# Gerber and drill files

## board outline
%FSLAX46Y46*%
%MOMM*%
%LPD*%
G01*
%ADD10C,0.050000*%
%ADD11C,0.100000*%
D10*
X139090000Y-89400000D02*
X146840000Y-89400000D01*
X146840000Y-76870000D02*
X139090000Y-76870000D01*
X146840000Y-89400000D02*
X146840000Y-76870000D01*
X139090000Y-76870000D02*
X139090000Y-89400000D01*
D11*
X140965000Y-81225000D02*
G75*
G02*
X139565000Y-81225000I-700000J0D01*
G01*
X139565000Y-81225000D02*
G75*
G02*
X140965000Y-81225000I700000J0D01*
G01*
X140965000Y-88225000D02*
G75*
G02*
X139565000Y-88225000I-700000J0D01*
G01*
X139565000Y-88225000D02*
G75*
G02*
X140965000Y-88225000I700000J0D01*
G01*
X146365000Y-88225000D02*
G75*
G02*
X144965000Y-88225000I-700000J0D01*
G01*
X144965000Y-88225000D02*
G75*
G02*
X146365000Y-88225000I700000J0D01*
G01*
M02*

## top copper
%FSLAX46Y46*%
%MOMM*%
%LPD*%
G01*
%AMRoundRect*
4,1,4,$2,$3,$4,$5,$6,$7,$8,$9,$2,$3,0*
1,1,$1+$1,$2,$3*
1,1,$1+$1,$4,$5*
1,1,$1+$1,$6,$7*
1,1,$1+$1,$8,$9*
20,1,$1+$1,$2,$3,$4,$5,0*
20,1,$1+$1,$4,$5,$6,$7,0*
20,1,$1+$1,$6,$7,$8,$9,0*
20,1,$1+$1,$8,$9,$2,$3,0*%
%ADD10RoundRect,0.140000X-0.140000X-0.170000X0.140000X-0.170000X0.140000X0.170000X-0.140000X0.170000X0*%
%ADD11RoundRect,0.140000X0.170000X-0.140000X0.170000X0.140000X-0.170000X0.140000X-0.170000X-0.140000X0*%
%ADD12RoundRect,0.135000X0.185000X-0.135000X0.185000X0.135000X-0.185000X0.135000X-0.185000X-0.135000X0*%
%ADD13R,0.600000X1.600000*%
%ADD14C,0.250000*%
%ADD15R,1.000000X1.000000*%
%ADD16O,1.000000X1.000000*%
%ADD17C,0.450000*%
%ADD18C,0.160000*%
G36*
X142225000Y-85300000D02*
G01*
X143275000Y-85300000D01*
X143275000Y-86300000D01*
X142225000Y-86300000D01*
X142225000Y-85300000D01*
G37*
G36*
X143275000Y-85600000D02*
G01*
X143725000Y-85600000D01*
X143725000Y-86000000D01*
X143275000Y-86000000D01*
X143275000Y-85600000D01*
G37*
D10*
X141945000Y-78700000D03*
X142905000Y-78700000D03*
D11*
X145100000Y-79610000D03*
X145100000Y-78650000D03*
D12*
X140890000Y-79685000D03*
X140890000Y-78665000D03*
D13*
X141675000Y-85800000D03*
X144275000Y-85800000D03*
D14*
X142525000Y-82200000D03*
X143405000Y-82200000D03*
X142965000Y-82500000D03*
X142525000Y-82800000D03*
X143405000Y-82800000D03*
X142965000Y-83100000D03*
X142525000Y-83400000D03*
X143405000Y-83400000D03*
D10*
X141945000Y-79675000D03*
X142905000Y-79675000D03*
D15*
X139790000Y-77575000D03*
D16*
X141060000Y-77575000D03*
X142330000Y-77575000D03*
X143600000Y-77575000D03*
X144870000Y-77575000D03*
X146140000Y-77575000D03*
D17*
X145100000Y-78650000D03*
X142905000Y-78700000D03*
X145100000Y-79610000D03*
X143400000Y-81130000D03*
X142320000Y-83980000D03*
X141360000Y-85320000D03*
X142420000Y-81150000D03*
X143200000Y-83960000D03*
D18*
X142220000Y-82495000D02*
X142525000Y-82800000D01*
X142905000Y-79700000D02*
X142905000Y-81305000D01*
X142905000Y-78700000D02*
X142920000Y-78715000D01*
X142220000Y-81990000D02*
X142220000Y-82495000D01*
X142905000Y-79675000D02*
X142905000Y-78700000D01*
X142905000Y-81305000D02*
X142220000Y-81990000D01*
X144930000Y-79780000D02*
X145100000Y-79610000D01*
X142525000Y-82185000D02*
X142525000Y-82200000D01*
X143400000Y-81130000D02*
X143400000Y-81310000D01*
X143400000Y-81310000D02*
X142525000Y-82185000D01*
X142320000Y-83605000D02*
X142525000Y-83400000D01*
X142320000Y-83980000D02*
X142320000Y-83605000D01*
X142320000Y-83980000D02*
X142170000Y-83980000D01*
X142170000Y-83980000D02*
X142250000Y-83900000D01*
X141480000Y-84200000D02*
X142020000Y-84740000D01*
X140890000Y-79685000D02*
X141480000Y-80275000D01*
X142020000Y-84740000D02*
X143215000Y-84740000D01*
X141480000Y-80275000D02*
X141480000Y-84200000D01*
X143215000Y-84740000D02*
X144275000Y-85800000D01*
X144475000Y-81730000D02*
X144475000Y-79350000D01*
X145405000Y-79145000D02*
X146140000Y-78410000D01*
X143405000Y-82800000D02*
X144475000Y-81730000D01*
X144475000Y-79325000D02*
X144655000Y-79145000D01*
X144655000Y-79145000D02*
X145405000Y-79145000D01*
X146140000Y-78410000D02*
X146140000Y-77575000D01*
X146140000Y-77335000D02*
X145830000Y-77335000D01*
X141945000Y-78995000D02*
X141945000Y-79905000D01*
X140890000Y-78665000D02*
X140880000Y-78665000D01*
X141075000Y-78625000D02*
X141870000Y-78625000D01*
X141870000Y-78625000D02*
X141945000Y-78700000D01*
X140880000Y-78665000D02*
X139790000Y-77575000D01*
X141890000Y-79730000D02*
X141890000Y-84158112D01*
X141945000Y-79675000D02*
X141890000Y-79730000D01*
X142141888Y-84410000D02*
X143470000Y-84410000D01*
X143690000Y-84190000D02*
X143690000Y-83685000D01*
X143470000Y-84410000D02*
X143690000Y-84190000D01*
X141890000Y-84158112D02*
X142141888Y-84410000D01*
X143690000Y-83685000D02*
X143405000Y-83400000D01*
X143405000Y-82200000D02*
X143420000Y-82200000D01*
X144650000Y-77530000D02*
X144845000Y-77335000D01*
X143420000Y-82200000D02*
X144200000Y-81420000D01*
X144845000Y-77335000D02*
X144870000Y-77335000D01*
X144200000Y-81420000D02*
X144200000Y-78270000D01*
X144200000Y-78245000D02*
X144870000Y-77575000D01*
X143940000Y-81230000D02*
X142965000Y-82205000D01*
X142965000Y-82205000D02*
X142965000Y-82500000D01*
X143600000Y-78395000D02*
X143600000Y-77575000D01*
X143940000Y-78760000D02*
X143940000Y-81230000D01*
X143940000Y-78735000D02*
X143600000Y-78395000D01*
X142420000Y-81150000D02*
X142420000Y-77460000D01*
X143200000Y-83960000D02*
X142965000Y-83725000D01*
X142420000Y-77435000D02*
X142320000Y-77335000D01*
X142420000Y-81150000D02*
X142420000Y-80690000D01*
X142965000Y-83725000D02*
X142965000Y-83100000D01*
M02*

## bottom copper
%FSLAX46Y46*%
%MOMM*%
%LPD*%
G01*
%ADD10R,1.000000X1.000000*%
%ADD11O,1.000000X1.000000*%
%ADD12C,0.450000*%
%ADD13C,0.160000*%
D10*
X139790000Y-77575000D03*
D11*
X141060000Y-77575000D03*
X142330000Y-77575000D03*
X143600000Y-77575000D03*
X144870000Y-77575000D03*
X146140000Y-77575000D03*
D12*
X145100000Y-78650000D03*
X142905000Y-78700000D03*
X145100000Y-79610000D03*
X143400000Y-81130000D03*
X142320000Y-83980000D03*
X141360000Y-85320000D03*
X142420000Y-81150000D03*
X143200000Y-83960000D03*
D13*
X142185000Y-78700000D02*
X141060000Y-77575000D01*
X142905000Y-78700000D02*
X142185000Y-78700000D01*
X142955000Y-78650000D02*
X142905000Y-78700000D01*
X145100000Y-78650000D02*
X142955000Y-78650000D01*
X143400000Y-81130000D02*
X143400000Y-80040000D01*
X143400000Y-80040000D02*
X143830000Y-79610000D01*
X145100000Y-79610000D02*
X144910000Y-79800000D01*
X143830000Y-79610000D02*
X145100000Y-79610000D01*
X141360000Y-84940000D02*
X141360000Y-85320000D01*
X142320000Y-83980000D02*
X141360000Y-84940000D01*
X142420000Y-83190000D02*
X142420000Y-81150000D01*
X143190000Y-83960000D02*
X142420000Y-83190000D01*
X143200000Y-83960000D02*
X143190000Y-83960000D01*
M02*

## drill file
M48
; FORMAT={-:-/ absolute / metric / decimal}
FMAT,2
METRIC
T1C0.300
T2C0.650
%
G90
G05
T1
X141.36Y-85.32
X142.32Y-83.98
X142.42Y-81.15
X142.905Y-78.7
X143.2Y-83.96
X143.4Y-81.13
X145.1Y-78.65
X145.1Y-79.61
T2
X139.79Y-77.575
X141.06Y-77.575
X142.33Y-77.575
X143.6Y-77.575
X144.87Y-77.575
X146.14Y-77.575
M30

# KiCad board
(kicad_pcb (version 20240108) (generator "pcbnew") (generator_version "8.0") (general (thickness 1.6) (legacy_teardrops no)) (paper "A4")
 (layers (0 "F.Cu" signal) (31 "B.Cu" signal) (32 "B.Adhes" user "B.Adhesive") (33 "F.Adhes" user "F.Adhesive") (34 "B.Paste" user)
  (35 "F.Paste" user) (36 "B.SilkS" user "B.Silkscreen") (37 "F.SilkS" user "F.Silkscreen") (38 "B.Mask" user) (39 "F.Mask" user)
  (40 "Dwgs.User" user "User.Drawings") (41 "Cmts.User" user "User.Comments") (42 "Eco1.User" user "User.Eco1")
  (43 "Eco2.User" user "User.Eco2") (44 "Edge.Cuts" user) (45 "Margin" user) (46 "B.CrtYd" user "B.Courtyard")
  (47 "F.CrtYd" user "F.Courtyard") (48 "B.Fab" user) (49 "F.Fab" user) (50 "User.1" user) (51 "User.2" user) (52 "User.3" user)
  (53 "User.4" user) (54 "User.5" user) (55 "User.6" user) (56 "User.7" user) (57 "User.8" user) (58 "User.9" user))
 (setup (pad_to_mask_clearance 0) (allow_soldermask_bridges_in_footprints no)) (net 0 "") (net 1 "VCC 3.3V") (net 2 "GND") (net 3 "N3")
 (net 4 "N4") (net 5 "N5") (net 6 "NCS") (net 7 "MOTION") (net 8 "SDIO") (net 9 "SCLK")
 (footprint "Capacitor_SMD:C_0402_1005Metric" (layer "F.Cu") (at 142.425 78.7)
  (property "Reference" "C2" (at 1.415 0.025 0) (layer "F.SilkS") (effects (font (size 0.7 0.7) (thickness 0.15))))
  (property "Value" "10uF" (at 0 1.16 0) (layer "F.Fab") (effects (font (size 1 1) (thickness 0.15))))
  (pad "1" smd roundrect (at -0.48 0) (size 0.56 0.62) (layers "F.Cu" "F.Paste" "F.Mask") (roundrect_rratio 0.25) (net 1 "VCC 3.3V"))
  (pad "2" smd roundrect (at 0.48 0) (size 0.56 0.62) (layers "F.Cu" "F.Paste" "F.Mask") (roundrect_rratio 0.25) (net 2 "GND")))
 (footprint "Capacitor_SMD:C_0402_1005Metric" (layer "F.Cu") (at 145.1 79.13 90)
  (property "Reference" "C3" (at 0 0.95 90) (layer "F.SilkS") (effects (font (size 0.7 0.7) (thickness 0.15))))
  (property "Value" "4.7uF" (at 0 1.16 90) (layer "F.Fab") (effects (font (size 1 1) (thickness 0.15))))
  (pad "1" smd roundrect (at -0.48 0 90) (size 0.56 0.62) (layers "F.Cu" "F.Paste" "F.Mask") (roundrect_rratio 0.25) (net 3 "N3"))
  (pad "2" smd roundrect (at 0.48 0 90) (size 0.56 0.62) (layers "F.Cu" "F.Paste" "F.Mask") (roundrect_rratio 0.25) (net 2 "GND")))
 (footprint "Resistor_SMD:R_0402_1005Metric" (layer "F.Cu") (at 140.89 79.175 90)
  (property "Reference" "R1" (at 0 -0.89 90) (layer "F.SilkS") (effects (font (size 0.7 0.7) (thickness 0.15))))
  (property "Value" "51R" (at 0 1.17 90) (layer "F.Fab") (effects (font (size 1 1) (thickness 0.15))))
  (pad "1" smd roundrect (at -0.51 0 90) (size 0.54 0.64) (layers "F.Cu" "F.Paste" "F.Mask") (roundrect_rratio 0.25) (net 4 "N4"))
  (pad "2" smd roundrect (at 0.51 0 90) (size 0.54 0.64) (layers "F.Cu" "F.Paste" "F.Mask") (roundrect_rratio 0.25) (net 1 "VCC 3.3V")))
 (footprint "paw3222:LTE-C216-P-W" (layer "F.Cu") (at 142.975 85.8 90)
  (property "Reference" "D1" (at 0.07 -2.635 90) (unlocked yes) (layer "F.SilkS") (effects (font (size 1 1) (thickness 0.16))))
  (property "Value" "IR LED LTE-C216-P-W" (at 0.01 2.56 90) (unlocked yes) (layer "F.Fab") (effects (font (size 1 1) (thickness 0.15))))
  (fp_rect (start -0.5 -0.75) (end 0.5 0.3) (stroke (width 0) (type solid)) (fill solid) (layer "F.Cu"))
  (fp_rect (start -0.2 0.3) (end 0.2 0.75) (stroke (width 0) (type solid)) (fill solid) (layer "F.Cu"))
  (pad "1" smd rect (at 0 -1.3 90) (size 1.6 0.6) (layers "F.Cu" "F.Paste" "F.Mask") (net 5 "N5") (thermal_bridge_angle 45))
  (pad "2" smd rect (at 0 1.3 90) (size 1.6 0.6) (layers "F.Cu" "F.Paste" "F.Mask") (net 4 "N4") (thermal_bridge_angle 45)))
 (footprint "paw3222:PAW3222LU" (layer "F.Cu") (at 142.965 82.8)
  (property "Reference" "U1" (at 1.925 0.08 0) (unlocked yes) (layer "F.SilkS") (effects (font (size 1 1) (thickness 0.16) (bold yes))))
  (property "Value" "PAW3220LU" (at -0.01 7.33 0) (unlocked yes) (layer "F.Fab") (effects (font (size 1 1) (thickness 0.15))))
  (fp_circle (center -2.7 -1.575) (end -2 -1.575) (stroke (width 0.1) (type default)) (fill none) (layer "Edge.Cuts"))
  (fp_circle (center -2.7 5.425) (end -2 5.425) (stroke (width 0.1) (type default)) (fill none) (layer "Edge.Cuts"))
  (fp_circle (center 2.7 5.425) (end 3.4 5.425) (stroke (width 0.1) (type default)) (fill none) (layer "Edge.Cuts"))
  (pad "A1" smd circle (at -0.44 -0.6) (size 0.25 0.25) (layers "F.Cu" "F.Paste" "F.Mask") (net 3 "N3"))
  (pad "A3" smd circle (at 0.44 -0.6) (size 0.25 0.25) (layers "F.Cu" "F.Paste" "F.Mask") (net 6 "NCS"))
  (pad "B2" smd circle (at 0 -0.3) (size 0.25 0.25) (layers "F.Cu" "F.Paste" "F.Mask") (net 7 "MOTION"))
  (pad "C1" smd circle (at -0.44 0) (size 0.25 0.25) (layers "F.Cu" "F.Paste" "F.Mask") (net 2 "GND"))
  (pad "C3" smd circle (at 0.44 0) (size 0.25 0.25) (layers "F.Cu" "F.Paste" "F.Mask") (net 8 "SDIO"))
  (pad "D2" smd circle (at 0 0.3) (size 0.25 0.25) (layers "F.Cu" "F.Paste" "F.Mask") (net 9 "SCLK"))
  (pad "E1" smd circle (at -0.44 0.6) (size 0.25 0.25) (layers "F.Cu" "F.Paste" "F.Mask") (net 5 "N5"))
  (pad "E3" smd circle (at 0.44 0.6) (size 0.25 0.25) (layers "F.Cu" "F.Paste" "F.Mask") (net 1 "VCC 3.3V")))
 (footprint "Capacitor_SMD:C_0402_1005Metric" (layer "F.Cu") (at 142.425 79.675)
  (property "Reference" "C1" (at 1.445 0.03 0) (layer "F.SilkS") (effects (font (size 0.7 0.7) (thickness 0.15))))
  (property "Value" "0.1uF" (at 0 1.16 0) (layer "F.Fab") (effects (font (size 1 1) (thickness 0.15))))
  (pad "1" smd roundrect (at -0.48 0) (size 0.56 0.62) (layers "F.Cu" "F.Paste" "F.Mask") (roundrect_rratio 0.25) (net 1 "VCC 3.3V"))
  (pad "2" smd roundrect (at 0.48 0) (size 0.56 0.62) (layers "F.Cu" "F.Paste" "F.Mask") (roundrect_rratio 0.25) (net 2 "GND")))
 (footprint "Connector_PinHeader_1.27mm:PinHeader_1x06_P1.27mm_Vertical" (layer "F.Cu") (at 139.79 77.575 90)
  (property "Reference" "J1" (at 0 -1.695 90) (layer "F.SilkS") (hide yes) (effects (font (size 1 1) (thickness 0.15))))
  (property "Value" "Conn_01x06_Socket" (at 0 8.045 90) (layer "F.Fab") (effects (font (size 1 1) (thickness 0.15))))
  (pad "1" thru_hole rect (at 0 0 90) (size 1 1) (drill 0.65) (layers "*.Cu" "*.Mask") (remove_unused_layers no) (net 1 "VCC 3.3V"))
  (pad "2" thru_hole oval (at 0 1.27 90) (size 1 1) (drill 0.65) (layers "*.Cu" "*.Mask") (remove_unused_layers no) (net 2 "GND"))
  (pad "3" thru_hole oval (at 0 2.54 90) (size 1 1) (drill 0.65) (layers "*.Cu" "*.Mask") (remove_unused_layers no) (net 9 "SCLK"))
  (pad "4" thru_hole oval (at 0 3.81 90) (size 1 1) (drill 0.65) (layers "*.Cu" "*.Mask") (remove_unused_layers no) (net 7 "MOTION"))
  (pad "5" thru_hole oval (at 0 5.08 90) (size 1 1) (drill 0.65) (layers "*.Cu" "*.Mask") (remove_unused_layers no) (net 6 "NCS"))
  (pad "6" thru_hole oval (at 0 6.35 90) (size 1 1) (drill 0.65) (layers "*.Cu" "*.Mask") (remove_unused_layers no) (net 8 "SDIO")))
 (gr_line (start 139.09 89.4) (end 146.84 89.4) (stroke (width 0.05) (type default)) (layer "Edge.Cuts"))
 (gr_line (start 146.84 76.87) (end 139.09 76.87) (stroke (width 0.05) (type default)) (layer "Edge.Cuts"))
 (gr_line (start 146.84 89.4) (end 146.84 76.87) (stroke (width 0.05) (type default)) (layer "Edge.Cuts"))
 (gr_line (start 139.09 76.87) (end 139.09 89.4) (stroke (width 0.05) (type default)) (layer "Edge.Cuts"))
 (segment (start 142.22 82.495) (end 142.525 82.8) (width 0.16) (layer "F.Cu") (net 2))
 (segment (start 142.905 79.7) (end 142.905 81.305) (width 0.16) (layer "F.Cu") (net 2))
 (segment (start 142.905 78.7) (end 142.92 78.715) (width 0.16) (layer "F.Cu") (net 2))
 (segment (start 142.22 81.99) (end 142.22 82.495) (width 0.16) (layer "F.Cu") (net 2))
 (segment (start 142.905 79.675) (end 142.905 78.7) (width 0.16) (layer "F.Cu") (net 2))
 (segment (start 142.905 81.305) (end 142.22 81.99) (width 0.16) (layer "F.Cu") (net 2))
 (via (at 145.1 78.65) (size 0.45) (drill 0.3) (layers "F.Cu" "B.Cu") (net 2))
 (via (at 142.905 78.7) (size 0.45) (drill 0.3) (layers "F.Cu" "B.Cu") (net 2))
 (segment (start 142.185 78.7) (end 141.06 77.575) (width 0.16) (layer "B.Cu") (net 2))
 (segment (start 142.905 78.7) (end 142.185 78.7) (width 0.16) (layer "B.Cu") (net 2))
 (segment (start 142.955 78.65) (end 142.905 78.7) (width 0.16) (layer "B.Cu") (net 2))
 (segment (start 145.1 78.65) (end 142.955 78.65) (width 0.16) (layer "B.Cu") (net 2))
 (segment (start 144.93 79.78) (end 145.1 79.61) (width 0.16) (layer "F.Cu") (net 3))
 (segment (start 142.525 82.185) (end 142.525 82.2) (width 0.16) (layer "F.Cu") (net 3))
 (segment (start 143.4 81.13) (end 143.4 81.31) (width 0.16) (layer "F.Cu") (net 3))
 (segment (start 143.4 81.31) (end 142.525 82.185) (width 0.16) (layer "F.Cu") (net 3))
 (via (at 145.1 79.61) (size 0.45) (drill 0.3) (layers "F.Cu" "B.Cu") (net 3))
 (via (at 143.4 81.13) (size 0.45) (drill 0.3) (layers "F.Cu" "B.Cu") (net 3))
 (segment (start 143.4 81.13) (end 143.4 80.04) (width 0.16) (layer "B.Cu") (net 3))
 (segment (start 143.4 80.04) (end 143.83 79.61) (width 0.16) (layer "B.Cu") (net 3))
 (segment (start 145.1 79.61) (end 144.91 79.8) (width 0.16) (layer "B.Cu") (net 3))
 (segment (start 143.83 79.61) (end 145.1 79.61) (width 0.16) (layer "B.Cu") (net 3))
 (segment (start 142.32 83.605) (end 142.525 83.4) (width 0.16) (layer "F.Cu") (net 5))
 (segment (start 142.32 83.98) (end 142.32 83.605) (width 0.16) (layer "F.Cu") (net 5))
 (segment (start 142.32 83.98) (end 142.17 83.98) (width 0.16) (layer "F.Cu") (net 5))
 (segment (start 142.17 83.98) (end 142.25 83.9) (width 0.16) (layer "F.Cu") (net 5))
 (via (at 142.32 83.98) (size 0.45) (drill 0.3) (layers "F.Cu" "B.Cu") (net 5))
 (via (at 141.36 85.32) (size 0.45) (drill 0.3) (layers "F.Cu" "B.Cu") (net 5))
 (segment (start 141.36 84.94) (end 141.36 85.32) (width 0.16) (layer "B.Cu") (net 5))
 (segment (start 142.32 83.98) (end 141.36 84.94) (width 0.16) (layer "B.Cu") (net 5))
 (segment (start 141.48 84.2) (end 142.02 84.74) (width 0.16) (layer "F.Cu") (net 4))
 (segment (start 140.89 79.685) (end 141.48 80.275) (width 0.16) (layer "F.Cu") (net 4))
 (segment (start 142.02 84.74) (end 143.215 84.74) (width 0.16) (layer "F.Cu") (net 4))
 (segment (start 141.48 80.275) (end 141.48 84.2) (width 0.16) (layer "F.Cu") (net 4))
 (segment (start 143.215 84.74) (end 144.275 85.8) (width 0.16) (layer "F.Cu") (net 4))
 (segment (start 144.475 81.73) (end 144.475 79.35) (width 0.16) (layer "F.Cu") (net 8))
 (segment (start 145.405 79.145) (end 146.14 78.41) (width 0.16) (layer "F.Cu") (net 8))
 (segment (start 143.405 82.8) (end 144.475 81.73) (width 0.16) (layer "F.Cu") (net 8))
 (segment (start 144.475 79.325) (end 144.655 79.145) (width 0.16) (layer "F.Cu") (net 8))
 (segment (start 144.655 79.145) (end 145.405 79.145) (width 0.16) (layer "F.Cu") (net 8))
 (segment (start 146.14 78.41) (end 146.14 77.575) (width 0.16) (layer "F.Cu") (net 8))
 (segment (start 146.14 77.335) (end 145.83 77.335) (width 0.16) (layer "F.Cu") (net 8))
 (segment (start 141.945 78.995) (end 141.945 79.905) (width 0.16) (layer "F.Cu") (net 1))
 (segment (start 140.89 78.665) (end 140.88 78.665) (width 0.16) (layer "F.Cu") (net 1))
 (segment (start 141.075 78.625) (end 141.87 78.625) (width 0.16) (layer "F.Cu") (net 1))
 (segment (start 141.87 78.625) (end 141.945 78.7) (width 0.16) (layer "F.Cu") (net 1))
 (segment (start 140.88 78.665) (end 139.79 77.575) (width 0.16) (layer "F.Cu") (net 1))
 (segment (start 141.89 79.73) (end 141.89 84.158112) (width 0.16) (layer "F.Cu") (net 1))
 (segment (start 141.945 79.675) (end 141.89 79.73) (width 0.16) (layer "F.Cu") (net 1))
 (segment (start 142.141888 84.41) (end 143.47 84.41) (width 0.16) (layer "F.Cu") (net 1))
 (segment (start 143.69 84.19) (end 143.69 83.685) (width 0.16) (layer "F.Cu") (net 1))
 (segment (start 143.47 84.41) (end 143.69 84.19) (width 0.16) (layer "F.Cu") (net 1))
 (segment (start 141.89 84.158112) (end 142.141888 84.41) (width 0.16) (layer "F.Cu") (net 1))
 (segment (start 143.69 83.685) (end 143.405 83.4) (width 0.16) (layer "F.Cu") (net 1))
 (segment (start 143.405 82.2) (end 143.42 82.2) (width 0.16) (layer "F.Cu") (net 6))
 (segment (start 144.65 77.53) (end 144.845 77.335) (width 0.16) (layer "F.Cu") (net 6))
 (segment (start 143.42 82.2) (end 144.2 81.42) (width 0.16) (layer "F.Cu") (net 6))
 (segment (start 144.845 77.335) (end 144.87 77.335) (width 0.16) (layer "F.Cu") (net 6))
 (segment (start 144.2 81.42) (end 144.2 78.27) (width 0.16) (layer "F.Cu") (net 6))
 (segment (start 144.2 78.245) (end 144.87 77.575) (width 0.16) (layer "F.Cu") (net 6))
 (segment (start 143.94 81.23) (end 142.965 82.205) (width 0.16) (layer "F.Cu") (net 7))
 (segment (start 142.965 82.205) (end 142.965 82.5) (width 0.16) (layer "F.Cu") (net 7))
 (segment (start 143.6 78.395) (end 143.6 77.575) (width 0.16) (layer "F.Cu") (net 7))
 (segment (start 143.94 78.76) (end 143.94 81.23) (width 0.16) (layer "F.Cu") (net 7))
 (segment (start 143.94 78.735) (end 143.6 78.395) (width 0.16) (layer "F.Cu") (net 7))
 (segment (start 142.42 81.15) (end 142.42 77.46) (width 0.16) (layer "F.Cu") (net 9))
 (segment (start 143.2 83.96) (end 142.965 83.725) (width 0.16) (layer "F.Cu") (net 9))
 (segment (start 142.42 77.435) (end 142.32 77.335) (width 0.16) (layer "F.Cu") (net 9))
 (segment (start 142.42 81.15) (end 142.42 80.69) (width 0.16) (layer "F.Cu") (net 9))
 (segment (start 142.965 83.725) (end 142.965 83.1) (width 0.16) (layer "F.Cu") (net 9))
 (via (at 142.42 81.15) (size 0.45) (drill 0.3) (layers "F.Cu" "B.Cu") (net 9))
 (via (at 143.2 83.96) (size 0.45) (drill 0.3) (layers "F.Cu" "B.Cu") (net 9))
 (segment (start 142.42 83.19) (end 142.42 81.15) (width 0.16) (layer "B.Cu") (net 9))
 (segment (start 143.19 83.96) (end 142.42 83.19) (width 0.16) (layer "B.Cu") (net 9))
 (segment (start 143.2 83.96) (end 143.19 83.96) (width 0.16) (layer "B.Cu") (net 9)))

